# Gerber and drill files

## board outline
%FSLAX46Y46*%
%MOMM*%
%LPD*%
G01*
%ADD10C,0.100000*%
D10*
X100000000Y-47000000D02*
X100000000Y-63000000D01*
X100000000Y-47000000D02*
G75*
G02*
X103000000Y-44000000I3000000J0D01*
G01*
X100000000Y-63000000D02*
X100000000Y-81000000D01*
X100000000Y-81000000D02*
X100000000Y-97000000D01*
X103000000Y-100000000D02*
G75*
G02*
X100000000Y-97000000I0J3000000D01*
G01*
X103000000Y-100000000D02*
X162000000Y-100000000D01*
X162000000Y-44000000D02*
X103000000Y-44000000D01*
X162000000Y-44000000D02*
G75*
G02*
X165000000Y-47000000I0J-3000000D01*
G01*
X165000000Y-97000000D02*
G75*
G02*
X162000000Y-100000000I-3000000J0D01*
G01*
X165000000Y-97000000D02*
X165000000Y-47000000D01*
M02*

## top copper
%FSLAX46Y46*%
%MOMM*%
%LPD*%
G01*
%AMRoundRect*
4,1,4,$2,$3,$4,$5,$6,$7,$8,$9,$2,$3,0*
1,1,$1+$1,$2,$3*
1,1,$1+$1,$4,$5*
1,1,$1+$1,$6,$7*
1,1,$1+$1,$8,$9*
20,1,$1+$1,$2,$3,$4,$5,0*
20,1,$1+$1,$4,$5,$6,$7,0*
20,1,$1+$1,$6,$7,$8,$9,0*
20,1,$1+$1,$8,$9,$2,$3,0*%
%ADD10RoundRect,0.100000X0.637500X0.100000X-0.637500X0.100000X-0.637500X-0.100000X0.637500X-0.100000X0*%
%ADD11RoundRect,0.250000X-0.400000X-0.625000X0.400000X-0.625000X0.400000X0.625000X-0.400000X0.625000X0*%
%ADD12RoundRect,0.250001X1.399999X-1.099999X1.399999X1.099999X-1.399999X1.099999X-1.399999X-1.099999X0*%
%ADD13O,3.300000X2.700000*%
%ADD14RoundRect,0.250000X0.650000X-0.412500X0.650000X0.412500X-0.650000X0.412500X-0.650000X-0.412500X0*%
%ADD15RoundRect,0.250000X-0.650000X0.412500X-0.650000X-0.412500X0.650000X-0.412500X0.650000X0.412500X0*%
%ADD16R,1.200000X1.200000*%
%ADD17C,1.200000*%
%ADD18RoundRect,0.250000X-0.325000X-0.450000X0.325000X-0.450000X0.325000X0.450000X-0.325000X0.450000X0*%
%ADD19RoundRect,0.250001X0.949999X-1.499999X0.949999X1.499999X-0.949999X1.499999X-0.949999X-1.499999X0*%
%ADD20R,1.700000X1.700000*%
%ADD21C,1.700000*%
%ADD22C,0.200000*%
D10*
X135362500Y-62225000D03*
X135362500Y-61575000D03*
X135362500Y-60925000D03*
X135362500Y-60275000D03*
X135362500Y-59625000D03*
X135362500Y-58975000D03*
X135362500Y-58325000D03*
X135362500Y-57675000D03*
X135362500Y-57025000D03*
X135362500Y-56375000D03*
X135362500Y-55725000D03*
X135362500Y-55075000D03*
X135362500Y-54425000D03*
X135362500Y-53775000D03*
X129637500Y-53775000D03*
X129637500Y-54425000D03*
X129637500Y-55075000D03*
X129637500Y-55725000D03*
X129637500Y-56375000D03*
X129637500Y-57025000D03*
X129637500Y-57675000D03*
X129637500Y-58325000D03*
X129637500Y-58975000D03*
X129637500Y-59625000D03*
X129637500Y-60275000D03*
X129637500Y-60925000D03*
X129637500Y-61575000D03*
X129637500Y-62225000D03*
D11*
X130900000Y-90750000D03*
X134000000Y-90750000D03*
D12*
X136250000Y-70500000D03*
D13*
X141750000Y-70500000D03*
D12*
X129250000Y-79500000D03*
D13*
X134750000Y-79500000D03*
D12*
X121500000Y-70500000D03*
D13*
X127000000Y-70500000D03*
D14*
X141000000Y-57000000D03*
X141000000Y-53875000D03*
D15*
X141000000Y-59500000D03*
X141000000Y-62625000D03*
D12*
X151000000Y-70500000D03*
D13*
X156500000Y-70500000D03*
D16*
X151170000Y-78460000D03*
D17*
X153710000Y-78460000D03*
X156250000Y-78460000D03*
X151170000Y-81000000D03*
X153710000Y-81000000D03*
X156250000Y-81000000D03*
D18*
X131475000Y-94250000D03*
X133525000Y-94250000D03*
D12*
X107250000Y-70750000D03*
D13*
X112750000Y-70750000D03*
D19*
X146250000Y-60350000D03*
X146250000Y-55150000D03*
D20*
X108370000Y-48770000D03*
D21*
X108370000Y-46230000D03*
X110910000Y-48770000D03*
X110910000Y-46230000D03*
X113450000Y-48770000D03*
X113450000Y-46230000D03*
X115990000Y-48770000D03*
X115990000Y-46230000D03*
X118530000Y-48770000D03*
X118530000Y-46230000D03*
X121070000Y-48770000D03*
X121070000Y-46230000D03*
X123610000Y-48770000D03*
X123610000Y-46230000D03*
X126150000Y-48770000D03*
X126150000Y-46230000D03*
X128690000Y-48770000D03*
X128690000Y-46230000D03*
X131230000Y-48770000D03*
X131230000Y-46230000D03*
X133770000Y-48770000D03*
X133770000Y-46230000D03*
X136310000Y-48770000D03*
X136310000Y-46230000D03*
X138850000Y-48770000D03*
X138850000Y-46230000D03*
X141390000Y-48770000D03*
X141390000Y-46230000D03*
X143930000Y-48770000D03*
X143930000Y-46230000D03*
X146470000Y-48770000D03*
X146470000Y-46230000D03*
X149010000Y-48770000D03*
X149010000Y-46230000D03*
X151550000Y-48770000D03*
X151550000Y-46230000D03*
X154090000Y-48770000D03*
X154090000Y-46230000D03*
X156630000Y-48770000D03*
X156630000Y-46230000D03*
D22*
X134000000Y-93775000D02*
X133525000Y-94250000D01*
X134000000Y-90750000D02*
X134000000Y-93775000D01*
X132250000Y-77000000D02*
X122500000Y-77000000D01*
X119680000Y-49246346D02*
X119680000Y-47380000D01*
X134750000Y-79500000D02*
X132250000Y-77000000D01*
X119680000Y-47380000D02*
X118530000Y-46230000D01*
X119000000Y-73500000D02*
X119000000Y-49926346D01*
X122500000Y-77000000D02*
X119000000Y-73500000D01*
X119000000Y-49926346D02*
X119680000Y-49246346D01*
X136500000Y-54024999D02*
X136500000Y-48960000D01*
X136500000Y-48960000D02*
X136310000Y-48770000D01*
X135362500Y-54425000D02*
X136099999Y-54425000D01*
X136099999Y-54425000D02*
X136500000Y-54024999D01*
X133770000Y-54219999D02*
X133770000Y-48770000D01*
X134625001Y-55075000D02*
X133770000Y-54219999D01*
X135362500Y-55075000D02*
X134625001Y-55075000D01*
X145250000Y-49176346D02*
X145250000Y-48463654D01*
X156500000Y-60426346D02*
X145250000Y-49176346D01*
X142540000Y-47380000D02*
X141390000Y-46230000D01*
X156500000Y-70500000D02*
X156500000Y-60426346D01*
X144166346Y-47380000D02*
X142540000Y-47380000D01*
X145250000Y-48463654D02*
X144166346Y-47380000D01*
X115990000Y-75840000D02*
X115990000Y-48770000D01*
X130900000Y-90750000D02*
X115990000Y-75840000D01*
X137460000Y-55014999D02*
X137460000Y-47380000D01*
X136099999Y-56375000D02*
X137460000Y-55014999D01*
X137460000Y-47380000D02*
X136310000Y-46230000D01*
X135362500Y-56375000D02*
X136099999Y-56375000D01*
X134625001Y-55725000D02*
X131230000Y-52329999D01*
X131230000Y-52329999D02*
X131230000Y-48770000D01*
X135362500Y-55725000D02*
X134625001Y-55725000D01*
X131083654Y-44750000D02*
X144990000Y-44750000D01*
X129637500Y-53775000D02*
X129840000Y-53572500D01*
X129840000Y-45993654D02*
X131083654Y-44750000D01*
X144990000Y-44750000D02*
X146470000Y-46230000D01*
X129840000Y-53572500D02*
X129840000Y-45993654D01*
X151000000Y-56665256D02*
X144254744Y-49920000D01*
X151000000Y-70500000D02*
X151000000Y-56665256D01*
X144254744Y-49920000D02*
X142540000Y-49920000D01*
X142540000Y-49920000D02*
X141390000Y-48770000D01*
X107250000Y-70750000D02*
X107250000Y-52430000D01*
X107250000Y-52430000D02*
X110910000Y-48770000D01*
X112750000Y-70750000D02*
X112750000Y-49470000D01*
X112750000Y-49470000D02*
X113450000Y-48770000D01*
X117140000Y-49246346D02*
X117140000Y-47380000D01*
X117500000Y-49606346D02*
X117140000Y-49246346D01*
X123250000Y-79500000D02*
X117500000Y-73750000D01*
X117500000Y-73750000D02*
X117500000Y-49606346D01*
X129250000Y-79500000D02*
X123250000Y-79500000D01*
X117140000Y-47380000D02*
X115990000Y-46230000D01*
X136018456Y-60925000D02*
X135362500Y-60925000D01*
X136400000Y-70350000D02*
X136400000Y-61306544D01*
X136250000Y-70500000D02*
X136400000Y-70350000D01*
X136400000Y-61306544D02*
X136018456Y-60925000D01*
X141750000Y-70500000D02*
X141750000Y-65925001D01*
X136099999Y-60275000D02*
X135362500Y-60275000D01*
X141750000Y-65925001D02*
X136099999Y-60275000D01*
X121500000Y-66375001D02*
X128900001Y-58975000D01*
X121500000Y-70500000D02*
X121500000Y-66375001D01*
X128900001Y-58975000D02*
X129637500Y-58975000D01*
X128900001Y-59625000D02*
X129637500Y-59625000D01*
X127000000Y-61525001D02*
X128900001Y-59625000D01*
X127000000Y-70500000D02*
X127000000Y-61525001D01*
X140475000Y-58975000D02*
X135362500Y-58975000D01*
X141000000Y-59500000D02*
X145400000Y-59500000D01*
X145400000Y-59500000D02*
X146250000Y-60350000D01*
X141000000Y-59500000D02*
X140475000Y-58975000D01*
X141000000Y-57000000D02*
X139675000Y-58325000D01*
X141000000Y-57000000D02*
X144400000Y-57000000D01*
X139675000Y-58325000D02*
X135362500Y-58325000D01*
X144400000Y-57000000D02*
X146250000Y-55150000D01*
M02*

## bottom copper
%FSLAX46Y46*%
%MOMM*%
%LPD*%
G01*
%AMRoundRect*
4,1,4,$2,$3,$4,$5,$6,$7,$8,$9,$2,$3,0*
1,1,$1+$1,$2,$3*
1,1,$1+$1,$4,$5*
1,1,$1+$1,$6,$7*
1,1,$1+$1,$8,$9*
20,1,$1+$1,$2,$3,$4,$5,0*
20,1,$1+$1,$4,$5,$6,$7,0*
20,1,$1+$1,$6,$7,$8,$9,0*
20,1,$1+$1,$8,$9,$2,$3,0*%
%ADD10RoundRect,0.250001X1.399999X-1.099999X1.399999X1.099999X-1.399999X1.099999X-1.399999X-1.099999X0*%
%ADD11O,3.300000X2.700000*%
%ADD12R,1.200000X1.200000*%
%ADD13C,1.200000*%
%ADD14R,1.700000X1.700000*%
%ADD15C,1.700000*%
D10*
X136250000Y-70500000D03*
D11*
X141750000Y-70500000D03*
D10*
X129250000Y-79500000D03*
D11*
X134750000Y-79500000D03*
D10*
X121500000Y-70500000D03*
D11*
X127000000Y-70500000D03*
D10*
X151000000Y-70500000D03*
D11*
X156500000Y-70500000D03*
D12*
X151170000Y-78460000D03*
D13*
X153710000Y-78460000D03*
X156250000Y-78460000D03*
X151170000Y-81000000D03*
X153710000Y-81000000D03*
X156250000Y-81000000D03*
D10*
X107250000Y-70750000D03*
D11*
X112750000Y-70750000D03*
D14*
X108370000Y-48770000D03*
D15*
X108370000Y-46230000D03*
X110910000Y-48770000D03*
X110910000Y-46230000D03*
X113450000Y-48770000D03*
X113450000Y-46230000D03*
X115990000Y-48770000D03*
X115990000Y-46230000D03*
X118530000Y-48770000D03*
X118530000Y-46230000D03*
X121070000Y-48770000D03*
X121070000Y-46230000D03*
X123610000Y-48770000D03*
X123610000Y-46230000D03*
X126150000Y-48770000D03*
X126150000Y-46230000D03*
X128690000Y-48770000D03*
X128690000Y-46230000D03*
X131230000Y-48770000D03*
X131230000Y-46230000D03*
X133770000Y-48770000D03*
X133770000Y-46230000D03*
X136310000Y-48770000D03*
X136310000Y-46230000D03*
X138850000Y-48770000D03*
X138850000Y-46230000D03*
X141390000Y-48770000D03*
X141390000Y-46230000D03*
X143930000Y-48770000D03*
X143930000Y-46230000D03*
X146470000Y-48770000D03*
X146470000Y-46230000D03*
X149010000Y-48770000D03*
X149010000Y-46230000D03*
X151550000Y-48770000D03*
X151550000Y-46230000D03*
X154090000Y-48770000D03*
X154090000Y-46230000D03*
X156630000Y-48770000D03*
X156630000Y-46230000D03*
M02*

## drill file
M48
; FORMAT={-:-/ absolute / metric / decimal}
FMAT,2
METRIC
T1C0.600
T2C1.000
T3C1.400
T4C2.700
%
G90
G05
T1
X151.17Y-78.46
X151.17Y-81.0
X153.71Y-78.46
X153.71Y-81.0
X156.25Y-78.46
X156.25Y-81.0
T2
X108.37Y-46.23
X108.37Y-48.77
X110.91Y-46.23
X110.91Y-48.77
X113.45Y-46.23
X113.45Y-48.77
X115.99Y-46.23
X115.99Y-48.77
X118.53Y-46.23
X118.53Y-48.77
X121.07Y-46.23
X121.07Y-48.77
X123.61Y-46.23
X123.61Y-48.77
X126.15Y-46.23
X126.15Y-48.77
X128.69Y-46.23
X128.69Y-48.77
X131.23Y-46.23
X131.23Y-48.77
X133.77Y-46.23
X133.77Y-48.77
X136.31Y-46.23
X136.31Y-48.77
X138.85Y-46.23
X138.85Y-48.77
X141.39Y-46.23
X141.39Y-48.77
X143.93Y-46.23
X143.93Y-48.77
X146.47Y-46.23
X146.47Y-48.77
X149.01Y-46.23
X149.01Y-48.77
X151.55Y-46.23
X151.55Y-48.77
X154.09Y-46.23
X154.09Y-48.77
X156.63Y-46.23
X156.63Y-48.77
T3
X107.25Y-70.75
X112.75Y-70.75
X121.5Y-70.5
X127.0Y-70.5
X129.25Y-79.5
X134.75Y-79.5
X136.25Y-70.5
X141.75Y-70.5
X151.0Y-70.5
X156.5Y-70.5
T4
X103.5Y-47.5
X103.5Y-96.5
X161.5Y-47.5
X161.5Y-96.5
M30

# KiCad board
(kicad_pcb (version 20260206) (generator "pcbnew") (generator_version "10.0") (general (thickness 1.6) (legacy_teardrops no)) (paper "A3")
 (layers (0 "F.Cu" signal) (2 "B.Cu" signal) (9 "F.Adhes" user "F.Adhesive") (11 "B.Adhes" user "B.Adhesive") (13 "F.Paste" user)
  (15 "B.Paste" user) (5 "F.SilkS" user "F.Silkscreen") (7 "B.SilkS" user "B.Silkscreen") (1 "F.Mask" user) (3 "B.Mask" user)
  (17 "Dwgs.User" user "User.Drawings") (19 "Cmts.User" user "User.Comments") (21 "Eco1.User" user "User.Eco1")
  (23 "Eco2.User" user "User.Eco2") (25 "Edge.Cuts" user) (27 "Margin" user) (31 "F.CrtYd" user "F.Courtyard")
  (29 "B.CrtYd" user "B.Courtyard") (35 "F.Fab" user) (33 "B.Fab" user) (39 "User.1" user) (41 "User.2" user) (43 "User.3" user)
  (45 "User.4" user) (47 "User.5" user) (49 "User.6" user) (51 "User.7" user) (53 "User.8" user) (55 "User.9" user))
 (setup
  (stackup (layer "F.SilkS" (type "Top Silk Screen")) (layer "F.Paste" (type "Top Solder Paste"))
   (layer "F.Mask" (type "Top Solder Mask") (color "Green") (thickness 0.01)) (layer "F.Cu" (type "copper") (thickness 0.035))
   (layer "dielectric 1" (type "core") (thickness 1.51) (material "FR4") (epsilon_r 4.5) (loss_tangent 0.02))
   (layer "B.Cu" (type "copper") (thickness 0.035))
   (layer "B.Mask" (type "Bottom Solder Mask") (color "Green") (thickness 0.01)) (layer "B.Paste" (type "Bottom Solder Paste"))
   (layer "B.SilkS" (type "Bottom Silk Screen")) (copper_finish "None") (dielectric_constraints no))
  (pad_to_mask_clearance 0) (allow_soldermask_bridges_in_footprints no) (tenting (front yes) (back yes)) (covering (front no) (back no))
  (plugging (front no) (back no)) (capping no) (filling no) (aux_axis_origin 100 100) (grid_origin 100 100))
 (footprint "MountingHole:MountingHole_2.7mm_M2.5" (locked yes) (layer "F.Cu") (at 161.5 47.5)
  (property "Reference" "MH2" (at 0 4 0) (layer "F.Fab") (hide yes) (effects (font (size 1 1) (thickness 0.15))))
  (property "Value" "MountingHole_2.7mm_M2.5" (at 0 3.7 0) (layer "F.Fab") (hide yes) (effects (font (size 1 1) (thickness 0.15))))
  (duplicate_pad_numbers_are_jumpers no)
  (pad "" np_thru_hole circle (at 0 0) (size 2.7 2.7) (drill 2.7) (layers "*.Cu" "*.Mask")))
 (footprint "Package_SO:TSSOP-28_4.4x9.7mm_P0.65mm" (layer "F.Cu") (at 132.5 58 180)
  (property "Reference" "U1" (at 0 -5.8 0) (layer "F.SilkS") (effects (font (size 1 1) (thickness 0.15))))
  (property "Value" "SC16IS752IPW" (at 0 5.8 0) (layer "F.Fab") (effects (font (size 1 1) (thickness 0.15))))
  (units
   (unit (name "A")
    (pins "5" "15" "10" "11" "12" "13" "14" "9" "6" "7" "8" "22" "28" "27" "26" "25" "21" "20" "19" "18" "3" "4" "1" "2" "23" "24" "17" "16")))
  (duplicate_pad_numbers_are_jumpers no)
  (pad "1" smd roundrect (at -2.8625 -4.225 180) (size 1.475 0.4) (layers "F.Cu" "F.Mask" "F.Paste") (roundrect_rratio 0.25)
   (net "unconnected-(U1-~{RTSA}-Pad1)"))
  (pad "2" smd roundrect (at -2.8625 -3.575 180) (size 1.475 0.4) (layers "F.Cu" "F.Mask" "F.Paste") (roundrect_rratio 0.25)
   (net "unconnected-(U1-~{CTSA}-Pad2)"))
  (pad "3" smd roundrect (at -2.8625 -2.925 180) (size 1.475 0.4) (layers "F.Cu" "F.Mask" "F.Paste") (roundrect_rratio 0.25)
   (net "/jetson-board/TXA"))
  (pad "4" smd roundrect (at -2.8625 -2.275 180) (size 1.475 0.4) (layers "F.Cu" "F.Mask" "F.Paste") (roundrect_rratio 0.25)
   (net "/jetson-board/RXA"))
  (pad "5" smd roundrect (at -2.8625 -1.625 180) (size 1.475 0.4) (layers "F.Cu" "F.Mask" "F.Paste") (roundrect_rratio 0.25)
   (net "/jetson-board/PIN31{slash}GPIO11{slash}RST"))
  (pad "6" smd roundrect (at -2.8625 -0.975 180) (size 1.475 0.4) (layers "F.Cu" "F.Mask" "F.Paste") (roundrect_rratio 0.25)
   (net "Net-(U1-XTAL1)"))
  (pad "7" smd roundrect (at -2.8625 -0.325 180) (size 1.475 0.4) (layers "F.Cu" "F.Mask" "F.Paste") (roundrect_rratio 0.25)
   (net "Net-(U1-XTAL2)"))
  (pad "8" smd roundrect (at -2.8625 0.325 180) (size 1.475 0.4) (layers "F.Cu" "F.Mask" "F.Paste") (roundrect_rratio 0.25) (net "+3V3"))
  (pad "9" smd roundrect (at -2.8625 0.975 180) (size 1.475 0.4) (layers "F.Cu" "F.Mask" "F.Paste") (roundrect_rratio 0.25) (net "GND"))
  (pad "10" smd roundrect (at -2.8625 1.625 180) (size 1.475 0.4) (layers "F.Cu" "F.Mask" "F.Paste") (roundrect_rratio 0.25)
   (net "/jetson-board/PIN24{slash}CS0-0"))
  (pad "11" smd roundrect (at -2.8625 2.275 180) (size 1.475 0.4) (layers "F.Cu" "F.Mask" "F.Paste") (roundrect_rratio 0.25)
   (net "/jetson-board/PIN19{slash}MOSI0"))
  (pad "12" smd roundrect (at -2.8625 2.925 180) (size 1.475 0.4) (layers "F.Cu" "F.Mask" "F.Paste") (roundrect_rratio 0.25)
   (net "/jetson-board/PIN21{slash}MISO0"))
  (pad "13" smd roundrect (at -2.8625 3.575 180) (size 1.475 0.4) (layers "F.Cu" "F.Mask" "F.Paste") (roundrect_rratio 0.25)
   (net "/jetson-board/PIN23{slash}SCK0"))
  (pad "14" smd roundrect (at -2.8625 4.225 180) (size 1.475 0.4) (layers "F.Cu" "F.Mask" "F.Paste") (roundrect_rratio 0.25) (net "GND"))
  (pad "15" smd roundrect (at 2.8625 4.225 180) (size 1.475 0.4) (layers "F.Cu" "F.Mask" "F.Paste") (roundrect_rratio 0.25)
   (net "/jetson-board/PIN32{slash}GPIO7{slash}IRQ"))
  (pad "16" smd roundrect (at 2.8625 3.575 180) (size 1.475 0.4) (layers "F.Cu" "F.Mask" "F.Paste") (roundrect_rratio 0.25)
   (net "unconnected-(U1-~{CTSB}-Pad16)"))
  (pad "17" smd roundrect (at 2.8625 2.925 180) (size 1.475 0.4) (layers "F.Cu" "F.Mask" "F.Paste") (roundrect_rratio 0.25)
   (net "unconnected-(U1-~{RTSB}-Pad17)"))
  (pad "18" smd roundrect (at 2.8625 2.275 180) (size 1.475 0.4) (layers "F.Cu" "F.Mask" "F.Paste") (roundrect_rratio 0.25)
   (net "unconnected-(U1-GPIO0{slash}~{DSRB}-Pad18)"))
  (pad "19" smd roundrect (at 2.8625 1.625 180) (size 1.475 0.4) (layers "F.Cu" "F.Mask" "F.Paste") (roundrect_rratio 0.25)
   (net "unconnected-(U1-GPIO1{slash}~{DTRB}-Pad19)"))
  (pad "20" smd roundrect (at 2.8625 0.975 180) (size 1.475 0.4) (layers "F.Cu" "F.Mask" "F.Paste") (roundrect_rratio 0.25)
   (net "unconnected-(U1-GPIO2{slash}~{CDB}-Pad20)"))
  (pad "21" smd roundrect (at 2.8625 0.325 180) (size 1.475 0.4) (layers "F.Cu" "F.Mask" "F.Paste") (roundrect_rratio 0.25)
   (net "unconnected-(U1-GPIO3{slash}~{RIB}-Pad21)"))
  (pad "22" smd roundrect (at 2.8625 -0.325 180) (size 1.475 0.4) (layers "F.Cu" "F.Mask" "F.Paste") (roundrect_rratio 0.25) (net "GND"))
  (pad "23" smd roundrect (at 2.8625 -0.975 180) (size 1.475 0.4) (layers "F.Cu" "F.Mask" "F.Paste") (roundrect_rratio 0.25)
   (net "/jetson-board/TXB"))
  (pad "24" smd roundrect (at 2.8625 -1.625 180) (size 1.475 0.4) (layers "F.Cu" "F.Mask" "F.Paste") (roundrect_rratio 0.25)
   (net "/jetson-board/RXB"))
  (pad "25" smd roundrect (at 2.8625 -2.275 180) (size 1.475 0.4) (layers "F.Cu" "F.Mask" "F.Paste") (roundrect_rratio 0.25)
   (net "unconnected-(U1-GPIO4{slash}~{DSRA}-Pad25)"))
  (pad "26" smd roundrect (at 2.8625 -2.925 180) (size 1.475 0.4) (layers "F.Cu" "F.Mask" "F.Paste") (roundrect_rratio 0.25)
   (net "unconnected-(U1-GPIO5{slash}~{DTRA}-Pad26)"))
  (pad "27" smd roundrect (at 2.8625 -3.575 180) (size 1.475 0.4) (layers "F.Cu" "F.Mask" "F.Paste") (roundrect_rratio 0.25)
   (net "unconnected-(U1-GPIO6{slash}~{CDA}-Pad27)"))
  (pad "28" smd roundrect (at 2.8625 -4.225 180) (size 1.475 0.4) (layers "F.Cu" "F.Mask" "F.Paste") (roundrect_rratio 0.25)
   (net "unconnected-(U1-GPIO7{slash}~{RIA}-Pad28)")))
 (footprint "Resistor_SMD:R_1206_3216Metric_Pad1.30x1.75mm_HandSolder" (layer "F.Cu") (at 132.45 90.75)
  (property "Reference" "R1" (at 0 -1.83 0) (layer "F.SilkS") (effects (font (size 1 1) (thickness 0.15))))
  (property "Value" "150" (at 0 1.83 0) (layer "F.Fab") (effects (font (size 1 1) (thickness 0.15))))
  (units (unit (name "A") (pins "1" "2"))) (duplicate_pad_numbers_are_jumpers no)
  (pad "1" smd roundrect (at -1.55 0) (size 1.3 1.75) (layers "F.Cu" "F.Mask" "F.Paste") (roundrect_rratio 0.192308)
   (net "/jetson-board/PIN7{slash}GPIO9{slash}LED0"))
  (pad "2" smd roundrect (at 1.55 0) (size 1.3 1.75) (layers "F.Cu" "F.Mask" "F.Paste") (roundrect_rratio 0.192308) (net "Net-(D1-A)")))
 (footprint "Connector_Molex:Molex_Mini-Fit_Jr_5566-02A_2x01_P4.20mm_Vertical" (layer "F.Cu") (at 136.25 70.5 90)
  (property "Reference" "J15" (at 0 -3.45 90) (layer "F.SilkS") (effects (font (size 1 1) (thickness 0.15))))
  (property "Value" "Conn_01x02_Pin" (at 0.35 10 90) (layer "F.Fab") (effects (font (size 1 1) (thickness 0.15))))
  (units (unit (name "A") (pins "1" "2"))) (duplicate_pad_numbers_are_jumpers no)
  (pad "1" thru_hole roundrect (at 0 0 90) (size 2.7 3.3) (drill 1.4) (layers "*.Cu" "*.Mask") (remove_unused_layers no)
   (roundrect_rratio 0.092593) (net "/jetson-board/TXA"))
  (pad "2" thru_hole oval (at 0 5.5 90) (size 2.7 3.3) (drill 1.4) (layers "*.Cu" "*.Mask") (remove_unused_layers no)
   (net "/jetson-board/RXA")))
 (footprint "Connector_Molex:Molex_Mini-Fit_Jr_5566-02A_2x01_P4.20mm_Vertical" (layer "F.Cu") (at 129.25 79.5 90)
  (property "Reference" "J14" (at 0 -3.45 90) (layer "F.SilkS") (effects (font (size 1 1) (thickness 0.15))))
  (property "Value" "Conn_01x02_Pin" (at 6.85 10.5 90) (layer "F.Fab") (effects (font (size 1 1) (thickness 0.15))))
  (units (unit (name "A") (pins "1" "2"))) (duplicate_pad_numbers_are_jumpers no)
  (pad "1" thru_hole roundrect (at 0 0 90) (size 2.7 3.3) (drill 1.4) (layers "*.Cu" "*.Mask") (remove_unused_layers no)
   (roundrect_rratio 0.092593) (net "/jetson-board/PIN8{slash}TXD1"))
  (pad "2" thru_hole oval (at 0 5.5 90) (size 2.7 3.3) (drill 1.4) (layers "*.Cu" "*.Mask") (remove_unused_layers no)
   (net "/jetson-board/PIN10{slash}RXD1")))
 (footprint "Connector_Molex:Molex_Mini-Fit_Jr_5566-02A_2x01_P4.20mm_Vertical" (layer "F.Cu") (at 121.5 70.5 90)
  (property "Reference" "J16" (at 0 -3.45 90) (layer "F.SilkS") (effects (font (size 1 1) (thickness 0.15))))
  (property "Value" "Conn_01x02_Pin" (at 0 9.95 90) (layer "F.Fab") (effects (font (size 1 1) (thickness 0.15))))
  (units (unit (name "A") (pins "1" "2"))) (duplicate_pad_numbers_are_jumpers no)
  (pad "1" thru_hole roundrect (at 0 0 90) (size 2.7 3.3) (drill 1.4) (layers "*.Cu" "*.Mask") (remove_unused_layers no)
   (roundrect_rratio 0.092593) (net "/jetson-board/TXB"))
  (pad "2" thru_hole oval (at 0 5.5 90) (size 2.7 3.3) (drill 1.4) (layers "*.Cu" "*.Mask") (remove_unused_layers no)
   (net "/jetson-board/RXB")))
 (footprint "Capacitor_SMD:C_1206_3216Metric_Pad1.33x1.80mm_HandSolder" (layer "F.Cu") (at 141 55.4375 90)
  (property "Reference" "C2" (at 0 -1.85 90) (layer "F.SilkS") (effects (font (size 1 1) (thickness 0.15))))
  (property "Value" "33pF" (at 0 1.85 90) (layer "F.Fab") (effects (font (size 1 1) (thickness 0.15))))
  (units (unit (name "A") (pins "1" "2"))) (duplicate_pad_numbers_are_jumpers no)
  (pad "1" smd roundrect (at -1.5625 0 90) (size 1.325 1.8) (layers "F.Cu" "F.Mask" "F.Paste") (roundrect_rratio 0.188679)
   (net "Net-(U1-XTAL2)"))
  (pad "2" smd roundrect (at 1.5625 0 90) (size 1.325 1.8) (layers "F.Cu" "F.Mask" "F.Paste") (roundrect_rratio 0.188679) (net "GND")))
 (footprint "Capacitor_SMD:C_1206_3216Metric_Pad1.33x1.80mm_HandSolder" (layer "F.Cu") (at 141 61.0625 -90)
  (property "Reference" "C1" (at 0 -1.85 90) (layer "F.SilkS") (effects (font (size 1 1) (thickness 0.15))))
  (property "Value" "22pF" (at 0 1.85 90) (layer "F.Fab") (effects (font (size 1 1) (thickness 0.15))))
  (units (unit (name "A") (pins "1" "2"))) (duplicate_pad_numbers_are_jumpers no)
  (pad "1" smd roundrect (at -1.5625 0 270) (size 1.325 1.8) (layers "F.Cu" "F.Mask" "F.Paste") (roundrect_rratio 0.188679)
   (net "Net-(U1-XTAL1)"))
  (pad "2" smd roundrect (at 1.5625 0 270) (size 1.325 1.8) (layers "F.Cu" "F.Mask" "F.Paste") (roundrect_rratio 0.188679) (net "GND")))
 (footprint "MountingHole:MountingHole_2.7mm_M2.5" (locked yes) (layer "F.Cu") (at 103.5 96.5)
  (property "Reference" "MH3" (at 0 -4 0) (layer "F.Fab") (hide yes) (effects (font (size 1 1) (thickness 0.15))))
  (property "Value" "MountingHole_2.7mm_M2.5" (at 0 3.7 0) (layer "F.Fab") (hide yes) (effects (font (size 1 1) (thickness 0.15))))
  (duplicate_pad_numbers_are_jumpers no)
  (pad "" np_thru_hole circle (at 0 0) (size 2.7 2.7) (drill 2.7) (layers "*.Cu" "*.Mask")))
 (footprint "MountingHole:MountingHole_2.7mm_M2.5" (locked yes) (layer "F.Cu") (at 103.5 47.5)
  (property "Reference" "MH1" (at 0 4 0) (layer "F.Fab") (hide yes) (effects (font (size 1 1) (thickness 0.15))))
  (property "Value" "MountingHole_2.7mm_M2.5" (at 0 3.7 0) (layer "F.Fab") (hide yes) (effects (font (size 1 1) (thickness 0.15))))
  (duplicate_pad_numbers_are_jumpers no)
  (pad "" np_thru_hole circle (at 0 0) (size 2.7 2.7) (drill 2.7) (layers "*.Cu" "*.Mask")))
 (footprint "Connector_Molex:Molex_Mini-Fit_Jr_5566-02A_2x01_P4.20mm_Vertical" (layer "F.Cu") (at 151 70.5 90)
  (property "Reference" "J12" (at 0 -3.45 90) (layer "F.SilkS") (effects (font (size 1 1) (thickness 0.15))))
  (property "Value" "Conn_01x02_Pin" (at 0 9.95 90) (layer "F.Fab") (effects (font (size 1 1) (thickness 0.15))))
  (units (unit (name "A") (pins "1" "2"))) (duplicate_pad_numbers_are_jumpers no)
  (pad "1" thru_hole roundrect (at 0 0 90) (size 2.7 3.3) (drill 1.4) (layers "*.Cu" "*.Mask") (remove_unused_layers no)
   (roundrect_rratio 0.092593) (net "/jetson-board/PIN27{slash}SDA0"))
  (pad "2" thru_hole oval (at 0 5.5 90) (size 2.7 3.3) (drill 1.4) (layers "*.Cu" "*.Mask") (remove_unused_layers no)
   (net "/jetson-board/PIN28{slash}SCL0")))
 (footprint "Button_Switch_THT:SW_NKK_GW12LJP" (layer "F.Cu") (at 151.17 78.46)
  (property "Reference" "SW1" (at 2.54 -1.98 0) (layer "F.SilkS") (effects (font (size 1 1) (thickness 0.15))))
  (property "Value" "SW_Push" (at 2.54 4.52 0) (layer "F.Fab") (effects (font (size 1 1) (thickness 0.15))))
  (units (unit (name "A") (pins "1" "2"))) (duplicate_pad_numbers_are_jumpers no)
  (pad "1" thru_hole rect (at 0 0) (size 1.2 1.2) (drill 0.6) (layers "*.Cu" "*.Mask") (remove_unused_layers no)
   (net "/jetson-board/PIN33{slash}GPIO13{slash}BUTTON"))
  (pad "2" thru_hole circle (at 2.54 0) (size 1.2 1.2) (drill 0.6) (layers "*.Cu" "*.Mask") (remove_unused_layers no) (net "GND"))
  (pad "3" thru_hole circle (at 5.08 0) (size 1.2 1.2) (drill 0.6) (layers "*.Cu" "*.Mask") (remove_unused_layers no))
  (pad "4" thru_hole circle (at 0 2.54) (size 1.2 1.2) (drill 0.6) (layers "*.Cu" "*.Mask") (remove_unused_layers no))
  (pad "5" thru_hole circle (at 2.54 2.54) (size 1.2 1.2) (drill 0.6) (layers "*.Cu" "*.Mask") (remove_unused_layers no))
  (pad "6" thru_hole circle (at 5.08 2.54) (size 1.2 1.2) (drill 0.6) (layers "*.Cu" "*.Mask") (remove_unused_layers no)))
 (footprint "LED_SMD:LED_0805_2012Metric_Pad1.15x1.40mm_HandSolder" (layer "F.Cu") (at 132.5 94.25)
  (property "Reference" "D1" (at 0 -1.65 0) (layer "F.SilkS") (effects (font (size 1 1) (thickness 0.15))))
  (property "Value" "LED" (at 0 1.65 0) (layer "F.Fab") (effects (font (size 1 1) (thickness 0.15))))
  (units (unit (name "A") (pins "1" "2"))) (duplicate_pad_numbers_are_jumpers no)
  (pad "1" smd roundrect (at -1.025 0) (size 1.15 1.4) (layers "F.Cu" "F.Mask" "F.Paste") (roundrect_rratio 0.217391) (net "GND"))
  (pad "2" smd roundrect (at 1.025 0) (size 1.15 1.4) (layers "F.Cu" "F.Mask" "F.Paste") (roundrect_rratio 0.217391) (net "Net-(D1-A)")))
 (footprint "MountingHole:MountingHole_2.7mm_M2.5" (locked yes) (layer "F.Cu") (at 161.5 96.5)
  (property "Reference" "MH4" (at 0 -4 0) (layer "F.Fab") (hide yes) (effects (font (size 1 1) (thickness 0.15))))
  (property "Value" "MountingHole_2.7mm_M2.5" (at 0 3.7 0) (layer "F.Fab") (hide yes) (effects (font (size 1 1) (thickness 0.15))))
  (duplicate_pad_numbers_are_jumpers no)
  (pad "" np_thru_hole circle (at 0 0) (size 2.7 2.7) (drill 2.7) (layers "*.Cu" "*.Mask")))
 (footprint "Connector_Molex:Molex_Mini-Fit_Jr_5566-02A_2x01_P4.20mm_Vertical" (layer "F.Cu") (at 107.25 70.75 90)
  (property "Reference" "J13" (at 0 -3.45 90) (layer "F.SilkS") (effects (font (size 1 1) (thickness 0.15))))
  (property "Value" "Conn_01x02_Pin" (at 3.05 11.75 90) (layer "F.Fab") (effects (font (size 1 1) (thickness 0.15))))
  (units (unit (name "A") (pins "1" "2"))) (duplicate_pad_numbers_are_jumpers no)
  (pad "1" thru_hole roundrect (at 0 0 90) (size 2.7 3.3) (drill 1.4) (layers "*.Cu" "*.Mask") (remove_unused_layers no)
   (roundrect_rratio 0.092593) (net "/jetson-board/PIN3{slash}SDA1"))
  (pad "2" thru_hole oval (at 0 5.5 90) (size 2.7 3.3) (drill 1.4) (layers "*.Cu" "*.Mask") (remove_unused_layers no)
   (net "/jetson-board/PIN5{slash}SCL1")))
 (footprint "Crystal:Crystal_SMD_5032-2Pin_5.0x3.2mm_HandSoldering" (layer "F.Cu") (at 146.25 57.75 90)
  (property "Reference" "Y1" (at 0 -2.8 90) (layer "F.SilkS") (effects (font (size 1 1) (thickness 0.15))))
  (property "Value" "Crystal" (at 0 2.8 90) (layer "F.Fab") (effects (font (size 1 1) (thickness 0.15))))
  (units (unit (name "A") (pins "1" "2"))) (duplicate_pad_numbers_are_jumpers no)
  (pad "1" smd roundrect (at -2.6 0 90) (size 3.5 2.4) (layers "F.Cu" "F.Mask" "F.Paste") (roundrect_rratio 0.104167) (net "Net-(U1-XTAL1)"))
  (pad "2" smd roundrect (at 2.6 0 90) (size 3.5 2.4) (layers "F.Cu" "F.Mask" "F.Paste") (roundrect_rratio 0.104167) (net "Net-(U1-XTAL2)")))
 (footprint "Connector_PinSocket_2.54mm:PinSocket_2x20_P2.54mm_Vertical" (layer "B.Cu") (at 108.37 48.77 -90)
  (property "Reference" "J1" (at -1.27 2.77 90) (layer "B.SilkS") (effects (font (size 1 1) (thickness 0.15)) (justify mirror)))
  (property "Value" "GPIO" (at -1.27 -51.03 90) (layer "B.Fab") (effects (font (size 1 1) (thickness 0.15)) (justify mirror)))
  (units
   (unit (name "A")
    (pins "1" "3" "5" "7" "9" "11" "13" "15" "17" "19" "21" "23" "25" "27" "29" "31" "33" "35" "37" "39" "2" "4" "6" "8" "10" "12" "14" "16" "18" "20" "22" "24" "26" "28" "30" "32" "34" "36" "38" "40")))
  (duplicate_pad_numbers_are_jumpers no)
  (pad "1" thru_hole rect (at 0 0 270) (size 1.7 1.7) (drill 1) (layers "*.Cu" "*.Mask") (remove_unused_layers no) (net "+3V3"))
  (pad "2" thru_hole circle (at -2.54 0 270) (size 1.7 1.7) (drill 1) (layers "*.Cu" "*.Mask") (remove_unused_layers no)
   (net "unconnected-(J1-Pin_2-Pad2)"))
  (pad "3" thru_hole circle (at 0 -2.54 270) (size 1.7 1.7) (drill 1) (layers "*.Cu" "*.Mask") (remove_unused_layers no)
   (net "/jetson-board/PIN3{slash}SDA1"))
  (pad "4" thru_hole circle (at -2.54 -2.54 270) (size 1.7 1.7) (drill 1) (layers "*.Cu" "*.Mask") (remove_unused_layers no)
   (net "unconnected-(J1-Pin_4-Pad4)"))
  (pad "5" thru_hole circle (at 0 -5.08 270) (size 1.7 1.7) (drill 1) (layers "*.Cu" "*.Mask") (remove_unused_layers no)
   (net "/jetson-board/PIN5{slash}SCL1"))
  (pad "6" thru_hole circle (at -2.54 -5.08 270) (size 1.7 1.7) (drill 1) (layers "*.Cu" "*.Mask") (remove_unused_layers no) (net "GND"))
  (pad "7" thru_hole circle (at 0 -7.62 270) (size 1.7 1.7) (drill 1) (layers "*.Cu" "*.Mask") (remove_unused_layers no)
   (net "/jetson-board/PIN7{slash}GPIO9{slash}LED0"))
  (pad "8" thru_hole circle (at -2.54 -7.62 270) (size 1.7 1.7) (drill 1) (layers "*.Cu" "*.Mask") (remove_unused_layers no)
   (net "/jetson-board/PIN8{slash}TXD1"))
  (pad "9" thru_hole circle (at 0 -10.16 270) (size 1.7 1.7) (drill 1) (layers "*.Cu" "*.Mask") (remove_unused_layers no)
   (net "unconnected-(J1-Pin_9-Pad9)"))
  (pad "10" thru_hole circle (at -2.54 -10.16 270) (size 1.7 1.7) (drill 1) (layers "*.Cu" "*.Mask") (remove_unused_layers no)
   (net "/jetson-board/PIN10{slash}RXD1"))
  (pad "11" thru_hole circle (at 0 -12.7 270) (size 1.7 1.7) (drill 1) (layers "*.Cu" "*.Mask") (remove_unused_layers no)
   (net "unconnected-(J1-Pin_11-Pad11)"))
  (pad "12" thru_hole circle (at -2.54 -12.7 270) (size 1.7 1.7) (drill 1) (layers "*.Cu" "*.Mask") (remove_unused_layers no)
   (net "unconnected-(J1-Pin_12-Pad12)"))
  (pad "13" thru_hole circle (at 0 -15.24 270) (size 1.7 1.7) (drill 1) (layers "*.Cu" "*.Mask") (remove_unused_layers no)
   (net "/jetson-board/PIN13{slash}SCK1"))
  (pad "14" thru_hole circle (at -2.54 -15.24 270) (size 1.7 1.7) (drill 1) (layers "*.Cu" "*.Mask") (remove_unused_layers no)
   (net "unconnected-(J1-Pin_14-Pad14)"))
  (pad "15" thru_hole circle (at 0 -17.78 270) (size 1.7 1.7) (drill 1) (layers "*.Cu" "*.Mask") (remove_unused_layers no)
   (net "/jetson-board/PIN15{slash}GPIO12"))
  (pad "16" thru_hole circle (at -2.54 -17.78 270) (size 1.7 1.7) (drill 1) (layers "*.Cu" "*.Mask") (remove_unused_layers no)
   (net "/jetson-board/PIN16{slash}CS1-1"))
  (pad "17" thru_hole circle (at 0 -20.32 270) (size 1.7 1.7) (drill 1) (layers "*.Cu" "*.Mask") (remove_unused_layers no)
   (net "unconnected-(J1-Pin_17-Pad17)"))
  (pad "18" thru_hole circle (at -2.54 -20.32 270) (size 1.7 1.7) (drill 1) (layers "*.Cu" "*.Mask") (remove_unused_layers no)
   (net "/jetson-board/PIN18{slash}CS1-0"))
  (pad "19" thru_hole circle (at 0 -22.86 270) (size 1.7 1.7) (drill 1) (layers "*.Cu" "*.Mask") (remove_unused_layers no)
   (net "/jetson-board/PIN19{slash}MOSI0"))
  (pad "20" thru_hole circle (at -2.54 -22.86 270) (size 1.7 1.7) (drill 1) (layers "*.Cu" "*.Mask") (remove_unused_layers no)
   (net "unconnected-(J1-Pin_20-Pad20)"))
  (pad "21" thru_hole circle (at 0 -25.4 270) (size 1.7 1.7) (drill 1) (layers "*.Cu" "*.Mask") (remove_unused_layers no)
   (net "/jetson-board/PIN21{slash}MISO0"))
  (pad "22" thru_hole circle (at -2.54 -25.4 270) (size 1.7 1.7) (drill 1) (layers "*.Cu" "*.Mask") (remove_unused_layers no)
   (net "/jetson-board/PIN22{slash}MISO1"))
  (pad "23" thru_hole circle (at 0 -27.94 270) (size 1.7 1.7) (drill 1) (layers "*.Cu" "*.Mask") (remove_unused_layers no)
   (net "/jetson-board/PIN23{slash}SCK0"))
  (pad "24" thru_hole circle (at -2.54 -27.94 270) (size 1.7 1.7) (drill 1) (layers "*.Cu" "*.Mask") (remove_unused_layers no)
   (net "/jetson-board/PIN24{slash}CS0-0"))
  (pad "25" thru_hole circle (at 0 -30.48 270) (size 1.7 1.7) (drill 1) (layers "*.Cu" "*.Mask") (remove_unused_layers no)
   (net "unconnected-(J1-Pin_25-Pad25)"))
  (pad "26" thru_hole circle (at -2.54 -30.48 270) (size 1.7 1.7) (drill 1) (layers "*.Cu" "*.Mask") (remove_unused_layers no)
   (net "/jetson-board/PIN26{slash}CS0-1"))
  (pad "27" thru_hole circle (at 0 -33.02 270) (size 1.7 1.7) (drill 1) (layers "*.Cu" "*.Mask") (remove_unused_layers no)
   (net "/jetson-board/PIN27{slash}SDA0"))
  (pad "28" thru_hole circle (at -2.54 -33.02 270) (size 1.7 1.7) (drill 1) (layers "*.Cu" "*.Mask") (remove_unused_layers no)
   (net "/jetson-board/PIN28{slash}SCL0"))
  (pad "29" thru_hole circle (at 0 -35.56 270) (size 1.7 1.7) (drill 1) (layers "*.Cu" "*.Mask") (remove_unused_layers no)
   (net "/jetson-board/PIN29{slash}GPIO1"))
  (pad "30" thru_hole circle (at -2.54 -35.56 270) (size 1.7 1.7) (drill 1) (layers "*.Cu" "*.Mask") (remove_unused_layers no)
   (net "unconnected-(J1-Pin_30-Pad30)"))
  (pad "31" thru_hole circle (at 0 -38.1 270) (size 1.7 1.7) (drill 1) (layers "*.Cu" "*.Mask") (remove_unused_layers no)
   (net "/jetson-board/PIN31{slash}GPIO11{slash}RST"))
  (pad "32" thru_hole circle (at -2.54 -38.1 270) (size 1.7 1.7) (drill 1) (layers "*.Cu" "*.Mask") (remove_unused_layers no)
   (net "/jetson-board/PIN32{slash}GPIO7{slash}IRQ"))
  (pad "33" thru_hole circle (at 0 -40.64 270) (size 1.7 1.7) (drill 1) (layers "*.Cu" "*.Mask") (remove_unused_layers no)
   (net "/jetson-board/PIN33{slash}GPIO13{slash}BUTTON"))
  (pad "34" thru_hole circle (at -2.54 -40.64 270) (size 1.7 1.7) (drill 1) (layers "*.Cu" "*.Mask") (remove_unused_layers no)
   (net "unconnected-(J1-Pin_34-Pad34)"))
  (pad "35" thru_hole circle (at 0 -43.18 270) (size 1.7 1.7) (drill 1) (layers "*.Cu" "*.Mask") (remove_unused_layers no)
   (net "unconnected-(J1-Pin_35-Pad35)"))
  (pad "36" thru_hole circle (at -2.54 -43.18 270) (size 1.7 1.7) (drill 1) (layers "*.Cu" "*.Mask") (remove_unused_layers no)
   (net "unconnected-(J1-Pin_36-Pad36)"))
  (pad "37" thru_hole circle (at 0 -45.72 270) (size 1.7 1.7) (drill 1) (layers "*.Cu" "*.Mask") (remove_unused_layers no)
   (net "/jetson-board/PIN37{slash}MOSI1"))
  (pad "38" thru_hole circle (at -2.54 -45.72 270) (size 1.7 1.7) (drill 1) (layers "*.Cu" "*.Mask") (remove_unused_layers no)
   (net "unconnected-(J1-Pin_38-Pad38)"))
  (pad "39" thru_hole circle (at 0 -48.26 270) (size 1.7 1.7) (drill 1) (layers "*.Cu" "*.Mask") (remove_unused_layers no)
   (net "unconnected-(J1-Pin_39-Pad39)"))
  (pad "40" thru_hole circle (at -2.54 -48.26 270) (size 1.7 1.7) (drill 1) (layers "*.Cu" "*.Mask") (remove_unused_layers no)
   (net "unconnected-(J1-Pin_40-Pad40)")))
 (gr_line (start 100 47) (end 100 63) (stroke (width 0.1) (type solid)) (layer "Edge.Cuts"))
 (gr_arc (start 100 47) (mid 100.87868 44.87868) (end 103 44) (stroke (width 0.1) (type solid)) (layer "Edge.Cuts"))
 (gr_line (start 100 63) (end 100 81) (stroke (width 0.1) (type solid)) (layer "Edge.Cuts"))
 (gr_line (start 100 81) (end 100 97) (stroke (width 0.1) (type solid)) (layer "Edge.Cuts"))
 (gr_arc (start 103 100) (mid 100.87868 99.12132) (end 100 97) (stroke (width 0.1) (type solid)) (layer "Edge.Cuts"))
 (gr_line (start 103 100) (end 162 100) (stroke (width 0.1) (type solid)) (layer "Edge.Cuts"))
 (gr_line (start 162 44) (end 103 44) (stroke (width 0.1) (type solid)) (layer "Edge.Cuts"))
 (gr_arc (start 162 44) (mid 164.12132 44.87868) (end 165 47) (stroke (width 0.1) (type solid)) (layer "Edge.Cuts"))
 (gr_arc (start 165 97) (mid 164.12132 99.12132) (end 162 100) (stroke (width 0.1) (type solid)) (layer "Edge.Cuts"))
 (gr_line (start 165 97) (end 165 47) (stroke (width 0.1) (type solid)) (layer "Edge.Cuts"))
 (segment (start 134 93.775) (end 133.525 94.25) (width 0.2) (layer "F.Cu") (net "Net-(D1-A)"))
 (segment (start 134 90.75) (end 134 93.775) (width 0.2) (layer "F.Cu") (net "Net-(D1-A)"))
 (segment (start 132.25 77) (end 122.5 77) (width 0.2) (layer "F.Cu") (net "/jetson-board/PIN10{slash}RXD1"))
 (segment (start 119.68 49.246346) (end 119.68 47.38) (width 0.2) (layer "F.Cu") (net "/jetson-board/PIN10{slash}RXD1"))
 (segment (start 134.75 79.5) (end 132.25 77) (width 0.2) (layer "F.Cu") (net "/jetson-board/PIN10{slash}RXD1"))
 (segment (start 119.68 47.38) (end 118.53 46.23) (width 0.2) (layer "F.Cu") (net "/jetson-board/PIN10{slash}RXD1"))
 (segment (start 119 73.5) (end 119 49.926346) (width 0.2) (layer "F.Cu") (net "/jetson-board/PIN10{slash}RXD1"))
 (segment (start 122.5 77) (end 119 73.5) (width 0.2) (layer "F.Cu") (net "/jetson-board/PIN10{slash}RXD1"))
 (segment (start 119 49.926346) (end 119.68 49.246346) (width 0.2) (layer "F.Cu") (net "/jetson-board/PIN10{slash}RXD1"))
 (segment (start 136.5 54.024999) (end 136.5 48.96) (width 0.2) (layer "F.Cu") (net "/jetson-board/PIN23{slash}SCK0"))
 (segment (start 136.5 48.96) (end 136.31 48.77) (width 0.2) (layer "F.Cu") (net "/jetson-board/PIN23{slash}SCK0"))
 (segment (start 135.3625 54.425) (end 136.099999 54.425) (width 0.2) (layer "F.Cu") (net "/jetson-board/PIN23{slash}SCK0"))
 (segment (start 136.099999 54.425) (end 136.5 54.024999) (width 0.2) (layer "F.Cu") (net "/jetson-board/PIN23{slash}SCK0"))
 (segment (start 133.77 54.219999) (end 133.77 48.77) (width 0.2) (layer "F.Cu") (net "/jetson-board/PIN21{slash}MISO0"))
 (segment (start 134.625001 55.075) (end 133.77 54.219999) (width 0.2) (layer "F.Cu") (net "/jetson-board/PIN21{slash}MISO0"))
 (segment (start 135.3625 55.075) (end 134.625001 55.075) (width 0.2) (layer "F.Cu") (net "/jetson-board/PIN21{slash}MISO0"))
 (segment (start 145.25 49.176346) (end 145.25 48.463654) (width 0.2) (layer "F.Cu") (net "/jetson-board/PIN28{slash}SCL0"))
 (segment (start 156.5 60.426346) (end 145.25 49.176346) (width 0.2) (layer "F.Cu") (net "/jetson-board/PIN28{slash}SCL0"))
 (segment (start 142.54 47.38) (end 141.39 46.23) (width 0.2) (layer "F.Cu") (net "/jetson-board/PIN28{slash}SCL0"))
 (segment (start 156.5 70.5) (end 156.5 60.426346) (width 0.2) (layer "F.Cu") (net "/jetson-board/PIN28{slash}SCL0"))
 (segment (start 144.166346 47.38) (end 142.54 47.38) (width 0.2) (layer "F.Cu") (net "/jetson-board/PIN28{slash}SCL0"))
 (segment (start 145.25 48.463654) (end 144.166346 47.38) (width 0.2) (layer "F.Cu") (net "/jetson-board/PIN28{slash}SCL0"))
 (segment (start 115.99 75.84) (end 115.99 48.77) (width 0.2) (layer "F.Cu") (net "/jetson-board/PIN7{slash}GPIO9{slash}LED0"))
 (segment (start 130.9 90.75) (end 115.99 75.84) (width 0.2) (layer "F.Cu") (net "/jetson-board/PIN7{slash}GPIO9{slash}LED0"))
 (segment (start 137.46 55.014999) (end 137.46 47.38) (width 0.2) (layer "F.Cu") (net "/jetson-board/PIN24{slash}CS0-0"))
 (segment (start 136.099999 56.375) (end 137.46 55.014999) (width 0.2) (layer "F.Cu") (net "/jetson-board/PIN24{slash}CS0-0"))
 (segment (start 137.46 47.38) (end 136.31 46.23) (width 0.2) (layer "F.Cu") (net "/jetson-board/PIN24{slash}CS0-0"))
 (segment (start 135.3625 56.375) (end 136.099999 56.375) (width 0.2) (layer "F.Cu") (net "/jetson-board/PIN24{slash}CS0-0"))
 (segment (start 134.625001 55.725) (end 131.23 52.329999) (width 0.2) (layer "F.Cu") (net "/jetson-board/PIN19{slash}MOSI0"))
 (segment (start 131.23 52.329999) (end 131.23 48.77) (width 0.2) (layer "F.Cu") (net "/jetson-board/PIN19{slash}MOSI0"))
 (segment (start 135.3625 55.725) (end 134.625001 55.725) (width 0.2) (layer "F.Cu") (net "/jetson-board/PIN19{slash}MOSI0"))
 (segment (start 131.083654 44.75) (end 144.99 44.75) (width 0.2) (layer "F.Cu") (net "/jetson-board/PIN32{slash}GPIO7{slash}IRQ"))
 (segment (start 129.6375 53.775) (end 129.84 53.5725) (width 0.2) (layer "F.Cu") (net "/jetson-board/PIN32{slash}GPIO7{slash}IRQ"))
 (segment (start 129.84 45.993654) (end 131.083654 44.75) (width 0.2) (layer "F.Cu") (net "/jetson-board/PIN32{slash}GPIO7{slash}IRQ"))
 (segment (start 144.99 44.75) (end 146.47 46.23) (width 0.2) (layer "F.Cu") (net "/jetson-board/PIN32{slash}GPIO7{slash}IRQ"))
 (segment (start 129.84 53.5725) (end 129.84 45.993654) (width 0.2) (layer "F.Cu") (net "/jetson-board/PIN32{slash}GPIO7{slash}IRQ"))
 (segment (start 151 56.665256) (end 144.254744 49.92) (width 0.2) (layer "F.Cu") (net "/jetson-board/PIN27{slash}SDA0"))
 (segment (start 151 70.5) (end 151 56.665256) (width 0.2) (layer "F.Cu") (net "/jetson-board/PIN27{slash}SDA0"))
 (segment (start 144.254744 49.92) (end 142.54 49.92) (width 0.2) (layer "F.Cu") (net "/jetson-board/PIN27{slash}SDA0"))
 (segment (start 142.54 49.92) (end 141.39 48.77) (width 0.2) (layer "F.Cu") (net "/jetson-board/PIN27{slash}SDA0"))
 (segment (start 107.25 70.75) (end 107.25 52.43) (width 0.2) (layer "F.Cu") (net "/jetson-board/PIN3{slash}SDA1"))
 (segment (start 107.25 52.43) (end 110.91 48.77) (width 0.2) (layer "F.Cu") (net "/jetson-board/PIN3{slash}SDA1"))
 (segment (start 112.75 70.75) (end 112.75 49.47) (width 0.2) (layer "F.Cu") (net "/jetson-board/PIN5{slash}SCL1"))
 (segment (start 112.75 49.47) (end 113.45 48.77) (width 0.2) (layer "F.Cu") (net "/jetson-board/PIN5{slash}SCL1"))
 (segment (start 117.14 49.246346) (end 117.14 47.38) (width 0.2) (layer "F.Cu") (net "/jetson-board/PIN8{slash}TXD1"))
 (segment (start 117.5 49.606346) (end 117.14 49.246346) (width 0.2) (layer "F.Cu") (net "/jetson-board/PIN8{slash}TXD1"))
 (segment (start 123.25 79.5) (end 117.5 73.75) (width 0.2) (layer "F.Cu") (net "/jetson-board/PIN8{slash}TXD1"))
 (segment (start 117.5 73.75) (end 117.5 49.606346) (width 0.2) (layer "F.Cu") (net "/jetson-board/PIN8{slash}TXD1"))
 (segment (start 129.25 79.5) (end 123.25 79.5) (width 0.2) (layer "F.Cu") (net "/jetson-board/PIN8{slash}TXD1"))
 (segment (start 117.14 47.38) (end 115.99 46.23) (width 0.2) (layer "F.Cu") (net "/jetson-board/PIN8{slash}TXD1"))
 (segment (start 136.018456 60.925) (end 135.3625 60.925) (width 0.2) (layer "F.Cu") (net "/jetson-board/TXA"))
 (segment (start 136.4 70.35) (end 136.4 61.306544) (width 0.2) (layer "F.Cu") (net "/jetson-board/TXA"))
 (segment (start 136.25 70.5) (end 136.4 70.35) (width 0.2) (layer "F.Cu") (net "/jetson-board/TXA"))
 (segment (start 136.4 61.306544) (end 136.018456 60.925) (width 0.2) (layer "F.Cu") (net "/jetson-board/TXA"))
 (segment (start 141.75 70.5) (end 141.75 65.925001) (width 0.2) (layer "F.Cu") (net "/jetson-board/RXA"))
 (segment (start 136.099999 60.275) (end 135.3625 60.275) (width 0.2) (layer "F.Cu") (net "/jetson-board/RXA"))
 (segment (start 141.75 65.925001) (end 136.099999 60.275) (width 0.2) (layer "F.Cu") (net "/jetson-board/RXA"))
 (segment (start 121.5 66.375001) (end 128.900001 58.975) (width 0.2) (layer "F.Cu") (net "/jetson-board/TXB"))
 (segment (start 121.5 70.5) (end 121.5 66.375001) (width 0.2) (layer "F.Cu") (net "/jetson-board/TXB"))
 (segment (start 128.900001 58.975) (end 129.6375 58.975) (width 0.2) (layer "F.Cu") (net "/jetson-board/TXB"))
 (segment (start 128.900001 59.625) (end 129.6375 59.625) (width 0.2) (layer "F.Cu") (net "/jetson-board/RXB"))
 (segment (start 127 61.525001) (end 128.900001 59.625) (width 0.2) (layer "F.Cu") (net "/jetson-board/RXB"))
 (segment (start 127 70.5) (end 127 61.525001) (width 0.2) (layer "F.Cu") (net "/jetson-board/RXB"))
 (segment (start 140.475 58.975) (end 135.3625 58.975) (width 0.2) (layer "F.Cu") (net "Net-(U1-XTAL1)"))
 (segment (start 141 59.5) (end 145.4 59.5) (width 0.2) (layer "F.Cu") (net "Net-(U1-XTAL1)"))
 (segment (start 145.4 59.5) (end 146.25 60.35) (width 0.2) (layer "F.Cu") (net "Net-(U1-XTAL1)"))
 (segment (start 141 59.5) (end 140.475 58.975) (width 0.2) (layer "F.Cu") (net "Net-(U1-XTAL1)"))
 (segment (start 141 57) (end 139.675 58.325) (width 0.2) (layer "F.Cu") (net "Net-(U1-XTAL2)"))
 (segment (start 141 57) (end 144.4 57) (width 0.2) (layer "F.Cu") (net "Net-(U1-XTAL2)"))
 (segment (start 139.675 58.325) (end 135.3625 58.325) (width 0.2) (layer "F.Cu") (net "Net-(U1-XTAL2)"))
 (segment (start 144.4 57) (end 146.25 55.15) (width 0.2) (layer "F.Cu") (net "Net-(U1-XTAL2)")))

